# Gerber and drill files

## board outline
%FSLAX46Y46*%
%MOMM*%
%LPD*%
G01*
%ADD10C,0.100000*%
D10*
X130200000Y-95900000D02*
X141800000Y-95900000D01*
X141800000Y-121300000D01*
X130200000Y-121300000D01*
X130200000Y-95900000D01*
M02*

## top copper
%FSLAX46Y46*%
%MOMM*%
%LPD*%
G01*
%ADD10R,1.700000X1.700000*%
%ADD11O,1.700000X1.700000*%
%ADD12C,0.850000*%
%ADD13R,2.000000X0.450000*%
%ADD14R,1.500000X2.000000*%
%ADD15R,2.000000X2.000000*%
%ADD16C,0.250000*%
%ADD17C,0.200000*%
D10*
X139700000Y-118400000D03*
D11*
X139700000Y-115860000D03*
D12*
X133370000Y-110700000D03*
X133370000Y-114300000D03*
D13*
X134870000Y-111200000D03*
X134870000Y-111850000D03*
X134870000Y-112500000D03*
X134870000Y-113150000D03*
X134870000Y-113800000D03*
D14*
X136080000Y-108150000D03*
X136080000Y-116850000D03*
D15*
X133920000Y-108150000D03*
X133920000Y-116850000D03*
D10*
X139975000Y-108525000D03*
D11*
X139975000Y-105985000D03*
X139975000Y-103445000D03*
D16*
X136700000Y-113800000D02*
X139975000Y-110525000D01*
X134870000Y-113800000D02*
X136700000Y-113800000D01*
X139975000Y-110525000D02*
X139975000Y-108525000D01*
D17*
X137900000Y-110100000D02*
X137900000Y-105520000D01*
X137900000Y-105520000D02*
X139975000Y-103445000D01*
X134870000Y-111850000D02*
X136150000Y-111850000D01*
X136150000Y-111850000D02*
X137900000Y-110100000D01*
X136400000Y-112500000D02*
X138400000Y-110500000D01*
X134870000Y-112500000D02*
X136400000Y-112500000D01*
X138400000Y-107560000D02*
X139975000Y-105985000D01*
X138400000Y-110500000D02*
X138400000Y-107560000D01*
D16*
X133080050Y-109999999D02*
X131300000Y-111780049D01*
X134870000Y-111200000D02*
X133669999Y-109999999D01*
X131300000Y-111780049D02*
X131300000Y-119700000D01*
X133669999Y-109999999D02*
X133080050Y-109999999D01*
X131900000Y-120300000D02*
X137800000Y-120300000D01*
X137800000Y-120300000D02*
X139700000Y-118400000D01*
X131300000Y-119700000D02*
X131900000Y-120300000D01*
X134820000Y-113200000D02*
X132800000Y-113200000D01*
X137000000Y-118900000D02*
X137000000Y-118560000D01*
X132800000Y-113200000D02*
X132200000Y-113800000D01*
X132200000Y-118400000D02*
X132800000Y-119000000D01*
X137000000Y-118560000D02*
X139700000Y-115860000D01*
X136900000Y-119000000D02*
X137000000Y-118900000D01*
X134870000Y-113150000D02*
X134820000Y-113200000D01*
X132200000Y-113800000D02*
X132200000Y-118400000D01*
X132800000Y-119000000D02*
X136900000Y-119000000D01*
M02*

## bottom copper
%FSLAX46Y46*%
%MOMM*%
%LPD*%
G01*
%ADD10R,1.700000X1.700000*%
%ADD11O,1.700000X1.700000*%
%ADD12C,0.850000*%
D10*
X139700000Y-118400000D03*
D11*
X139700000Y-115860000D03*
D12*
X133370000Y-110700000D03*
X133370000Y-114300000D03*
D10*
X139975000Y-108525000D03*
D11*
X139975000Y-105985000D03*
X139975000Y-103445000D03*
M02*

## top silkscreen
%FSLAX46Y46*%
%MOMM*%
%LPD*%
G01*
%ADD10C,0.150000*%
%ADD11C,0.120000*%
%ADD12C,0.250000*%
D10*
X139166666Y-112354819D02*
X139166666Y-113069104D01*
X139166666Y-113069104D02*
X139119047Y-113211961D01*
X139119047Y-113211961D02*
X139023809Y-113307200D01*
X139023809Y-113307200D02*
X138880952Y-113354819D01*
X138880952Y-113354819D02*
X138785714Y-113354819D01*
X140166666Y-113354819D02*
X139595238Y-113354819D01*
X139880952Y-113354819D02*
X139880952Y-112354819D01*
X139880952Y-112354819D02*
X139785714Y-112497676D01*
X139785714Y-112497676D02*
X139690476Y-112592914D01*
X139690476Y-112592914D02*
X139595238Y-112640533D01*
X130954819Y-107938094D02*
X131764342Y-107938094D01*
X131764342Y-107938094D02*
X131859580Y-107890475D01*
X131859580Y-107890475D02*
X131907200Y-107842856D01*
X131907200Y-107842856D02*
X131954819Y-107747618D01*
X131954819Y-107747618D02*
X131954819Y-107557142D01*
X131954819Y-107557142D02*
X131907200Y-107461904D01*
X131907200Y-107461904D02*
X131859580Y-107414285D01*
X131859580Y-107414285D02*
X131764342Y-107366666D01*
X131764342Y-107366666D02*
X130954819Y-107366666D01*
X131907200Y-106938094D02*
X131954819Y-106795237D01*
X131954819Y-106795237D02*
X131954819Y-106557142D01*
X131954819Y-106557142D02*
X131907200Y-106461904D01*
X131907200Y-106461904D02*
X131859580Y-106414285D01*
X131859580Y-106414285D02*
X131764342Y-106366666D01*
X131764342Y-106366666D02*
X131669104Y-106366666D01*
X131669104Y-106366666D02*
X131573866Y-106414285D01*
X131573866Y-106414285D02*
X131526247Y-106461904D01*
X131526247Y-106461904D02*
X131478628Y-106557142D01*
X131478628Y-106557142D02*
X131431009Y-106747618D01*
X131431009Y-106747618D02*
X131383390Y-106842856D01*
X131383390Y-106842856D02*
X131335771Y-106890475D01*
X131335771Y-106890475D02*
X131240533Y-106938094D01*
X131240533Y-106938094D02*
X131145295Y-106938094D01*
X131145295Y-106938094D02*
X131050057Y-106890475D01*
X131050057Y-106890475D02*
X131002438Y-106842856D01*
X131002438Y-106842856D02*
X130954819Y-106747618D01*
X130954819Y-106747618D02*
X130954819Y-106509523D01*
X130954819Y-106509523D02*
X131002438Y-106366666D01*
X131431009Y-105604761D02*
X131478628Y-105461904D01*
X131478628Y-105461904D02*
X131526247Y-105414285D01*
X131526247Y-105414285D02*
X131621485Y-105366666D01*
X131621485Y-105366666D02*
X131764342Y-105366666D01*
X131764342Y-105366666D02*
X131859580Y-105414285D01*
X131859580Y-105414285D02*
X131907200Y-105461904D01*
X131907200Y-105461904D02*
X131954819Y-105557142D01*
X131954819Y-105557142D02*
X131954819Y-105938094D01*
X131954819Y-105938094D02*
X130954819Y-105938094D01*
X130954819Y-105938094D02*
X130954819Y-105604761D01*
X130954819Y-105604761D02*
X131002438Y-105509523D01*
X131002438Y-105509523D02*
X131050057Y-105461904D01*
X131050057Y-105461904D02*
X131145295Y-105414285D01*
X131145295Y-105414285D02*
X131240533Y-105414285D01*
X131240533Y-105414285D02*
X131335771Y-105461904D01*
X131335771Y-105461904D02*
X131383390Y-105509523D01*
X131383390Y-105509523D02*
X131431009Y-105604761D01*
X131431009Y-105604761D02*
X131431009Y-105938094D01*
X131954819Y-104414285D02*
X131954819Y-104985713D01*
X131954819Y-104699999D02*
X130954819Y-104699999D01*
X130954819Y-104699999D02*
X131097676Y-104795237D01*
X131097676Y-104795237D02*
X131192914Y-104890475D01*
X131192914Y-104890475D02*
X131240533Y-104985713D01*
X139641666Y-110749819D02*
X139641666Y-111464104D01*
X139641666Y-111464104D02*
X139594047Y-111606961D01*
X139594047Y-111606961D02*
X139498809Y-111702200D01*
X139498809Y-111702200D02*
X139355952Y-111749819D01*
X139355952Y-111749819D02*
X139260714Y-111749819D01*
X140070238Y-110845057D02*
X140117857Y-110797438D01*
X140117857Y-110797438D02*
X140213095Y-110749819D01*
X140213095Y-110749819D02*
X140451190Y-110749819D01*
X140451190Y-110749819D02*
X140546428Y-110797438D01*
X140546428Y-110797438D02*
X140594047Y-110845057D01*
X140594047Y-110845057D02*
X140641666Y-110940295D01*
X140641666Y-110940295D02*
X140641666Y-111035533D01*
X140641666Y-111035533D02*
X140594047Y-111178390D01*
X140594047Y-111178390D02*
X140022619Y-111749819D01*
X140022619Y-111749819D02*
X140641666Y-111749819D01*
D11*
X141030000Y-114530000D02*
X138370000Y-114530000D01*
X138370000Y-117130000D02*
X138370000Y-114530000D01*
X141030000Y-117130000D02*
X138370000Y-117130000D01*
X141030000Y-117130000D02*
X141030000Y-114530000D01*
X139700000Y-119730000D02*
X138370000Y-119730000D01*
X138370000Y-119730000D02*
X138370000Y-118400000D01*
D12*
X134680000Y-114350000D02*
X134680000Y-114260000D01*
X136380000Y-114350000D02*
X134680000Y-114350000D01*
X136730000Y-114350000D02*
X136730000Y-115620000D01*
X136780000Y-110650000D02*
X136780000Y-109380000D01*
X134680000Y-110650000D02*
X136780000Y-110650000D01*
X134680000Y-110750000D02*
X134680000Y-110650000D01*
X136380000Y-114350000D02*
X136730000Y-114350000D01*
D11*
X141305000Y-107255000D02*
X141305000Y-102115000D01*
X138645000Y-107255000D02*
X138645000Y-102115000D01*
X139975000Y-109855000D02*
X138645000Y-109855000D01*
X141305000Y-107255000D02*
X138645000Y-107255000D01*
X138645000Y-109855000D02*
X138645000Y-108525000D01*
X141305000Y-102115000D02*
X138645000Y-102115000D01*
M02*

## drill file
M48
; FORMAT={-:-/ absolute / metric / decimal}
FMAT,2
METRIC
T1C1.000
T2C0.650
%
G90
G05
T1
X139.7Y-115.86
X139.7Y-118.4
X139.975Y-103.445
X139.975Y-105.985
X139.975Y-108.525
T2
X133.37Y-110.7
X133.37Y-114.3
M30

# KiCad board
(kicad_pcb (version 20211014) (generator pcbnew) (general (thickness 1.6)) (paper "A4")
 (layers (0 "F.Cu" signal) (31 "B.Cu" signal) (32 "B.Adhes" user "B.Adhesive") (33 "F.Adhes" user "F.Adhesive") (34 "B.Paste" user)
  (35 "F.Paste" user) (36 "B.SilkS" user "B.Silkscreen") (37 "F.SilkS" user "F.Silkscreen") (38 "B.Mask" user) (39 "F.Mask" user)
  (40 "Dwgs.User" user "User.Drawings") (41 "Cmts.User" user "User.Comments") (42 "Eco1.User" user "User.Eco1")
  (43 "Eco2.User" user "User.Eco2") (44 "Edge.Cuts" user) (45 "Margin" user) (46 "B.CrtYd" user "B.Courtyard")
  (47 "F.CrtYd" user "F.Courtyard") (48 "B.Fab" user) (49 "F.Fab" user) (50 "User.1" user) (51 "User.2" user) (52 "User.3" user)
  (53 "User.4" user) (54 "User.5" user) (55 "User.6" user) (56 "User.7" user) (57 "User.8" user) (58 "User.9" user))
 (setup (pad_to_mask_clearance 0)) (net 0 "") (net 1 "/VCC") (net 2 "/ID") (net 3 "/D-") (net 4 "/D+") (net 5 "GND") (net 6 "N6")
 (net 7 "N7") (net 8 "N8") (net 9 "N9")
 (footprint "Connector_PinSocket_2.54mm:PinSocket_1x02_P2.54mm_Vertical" (layer "F.Cu") (at 139.7 118.4 180)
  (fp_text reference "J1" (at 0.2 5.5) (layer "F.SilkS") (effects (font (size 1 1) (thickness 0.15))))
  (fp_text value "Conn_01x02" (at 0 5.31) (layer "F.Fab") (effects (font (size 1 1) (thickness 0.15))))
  (fp_line (start -1.33 3.87) (end 1.33 3.87) (layer "F.SilkS") (width 0.12))
  (fp_line (start 1.33 1.27) (end 1.33 3.87) (layer "F.SilkS") (width 0.12))
  (fp_line (start -1.33 1.27) (end 1.33 1.27) (layer "F.SilkS") (width 0.12))
  (fp_line (start -1.33 1.27) (end -1.33 3.87) (layer "F.SilkS") (width 0.12))
  (fp_line (start 0 -1.33) (end 1.33 -1.33) (layer "F.SilkS") (width 0.12))
  (fp_line (start 1.33 -1.33) (end 1.33 0) (layer "F.SilkS") (width 0.12))
  (pad "1" thru_hole rect (at 0 0 180) (size 1.7 1.7) (drill 1) (layers *.Cu *.Mask) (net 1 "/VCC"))
  (pad "2" thru_hole oval (at 0 2.54 180) (size 1.7 1.7) (drill 1) (layers *.Cu *.Mask) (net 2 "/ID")))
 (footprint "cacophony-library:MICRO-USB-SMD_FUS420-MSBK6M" (layer "F.Cu") (at 135 112.5 -90)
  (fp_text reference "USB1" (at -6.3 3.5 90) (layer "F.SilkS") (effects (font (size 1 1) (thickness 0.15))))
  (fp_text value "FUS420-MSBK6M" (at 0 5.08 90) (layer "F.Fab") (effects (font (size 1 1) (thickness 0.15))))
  (fp_line (start 1.85 0.32) (end 1.76 0.32) (layer "F.SilkS") (width 0.25))
  (fp_line (start 1.85 -1.38) (end 1.85 0.32) (layer "F.SilkS") (width 0.25))
  (fp_line (start 1.85 -1.73) (end 3.12 -1.73) (layer "F.SilkS") (width 0.25))
  (fp_line (start -1.85 -1.78) (end -3.12 -1.78) (layer "F.SilkS") (width 0.25))
  (fp_line (start -1.85 0.32) (end -1.85 -1.78) (layer "F.SilkS") (width 0.25))
  (fp_line (start -1.75 0.32) (end -1.85 0.32) (layer "F.SilkS") (width 0.25))
  (fp_line (start 1.85 -1.38) (end 1.85 -1.73) (layer "F.SilkS") (width 0.25))
  (pad "" np_thru_hole circle (at -1.8 1.63 270) (size 0.85 0.85) (drill 0.65) (layers F&B.Cu *.Mask))
  (pad "" np_thru_hole circle (at 1.8 1.63 270) (size 0.85 0.85) (drill 0.65) (layers F&B.Cu *.Mask))
  (pad "1" smd rect (at -1.3 0.13 270) (size 0.45 2) (layers "F.Cu" "F.Paste" "F.Mask") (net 1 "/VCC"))
  (pad "2" smd rect (at -0.65 0.13 270) (size 0.45 2) (layers "F.Cu" "F.Paste" "F.Mask") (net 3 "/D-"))
  (pad "3" smd rect (at 0 0.13 270) (size 0.45 2) (layers "F.Cu" "F.Paste" "F.Mask") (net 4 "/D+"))
  (pad "4" smd rect (at 0.65 0.13 270) (size 0.45 2) (layers "F.Cu" "F.Paste" "F.Mask") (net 2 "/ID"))
  (pad "5" smd rect (at 1.3 0.13 270) (size 0.45 2) (layers "F.Cu" "F.Paste" "F.Mask") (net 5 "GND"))
  (pad "8" smd rect (at -4.35 -1.08 270) (size 2 1.5) (layers "F.Cu" "F.Paste" "F.Mask") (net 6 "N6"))
  (pad "9" smd rect (at 4.35 -1.08 270) (size 2 1.5) (layers "F.Cu" "F.Paste" "F.Mask") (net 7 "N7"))
  (pad "12" smd rect (at -4.35 1.08 270) (size 2 2) (layers "F.Cu" "F.Paste" "F.Mask") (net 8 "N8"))
  (pad "13" smd rect (at 4.35 1.08 270) (size 2 2) (layers "F.Cu" "F.Paste" "F.Mask") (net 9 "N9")))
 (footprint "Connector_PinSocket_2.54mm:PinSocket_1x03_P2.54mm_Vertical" (layer "F.Cu") (at 139.975 108.525 180)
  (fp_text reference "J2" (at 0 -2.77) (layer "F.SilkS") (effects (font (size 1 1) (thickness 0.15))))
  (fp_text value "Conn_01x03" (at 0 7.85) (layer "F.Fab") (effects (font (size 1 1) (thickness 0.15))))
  (fp_line (start -1.33 1.27) (end -1.33 6.41) (layer "F.SilkS") (width 0.12))
  (fp_line (start 1.33 1.27) (end 1.33 6.41) (layer "F.SilkS") (width 0.12))
  (fp_line (start 0 -1.33) (end 1.33 -1.33) (layer "F.SilkS") (width 0.12))
  (fp_line (start -1.33 1.27) (end 1.33 1.27) (layer "F.SilkS") (width 0.12))
  (fp_line (start 1.33 -1.33) (end 1.33 0) (layer "F.SilkS") (width 0.12))
  (fp_line (start -1.33 6.41) (end 1.33 6.41) (layer "F.SilkS") (width 0.12))
  (pad "1" thru_hole rect (at 0 0 180) (size 1.7 1.7) (drill 1) (layers *.Cu *.Mask) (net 5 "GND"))
  (pad "2" thru_hole oval (at 0 2.54 180) (size 1.7 1.7) (drill 1) (layers *.Cu *.Mask) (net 4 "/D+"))
  (pad "3" thru_hole oval (at 0 5.08 180) (size 1.7 1.7) (drill 1) (layers *.Cu *.Mask) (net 3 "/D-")))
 (gr_rect (start 130.2 121.3) (end 141.8 95.9) (layer "Edge.Cuts") (width 0.1) (fill none))
 (segment (start 136.7 113.8) (end 139.975 110.525) (width 0.25) (layer "F.Cu") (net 5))
 (segment (start 134.87 113.8) (end 136.7 113.8) (width 0.25) (layer "F.Cu") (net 5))
 (segment (start 139.975 110.525) (end 139.975 108.525) (width 0.25) (layer "F.Cu") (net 5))
 (segment (start 137.9 110.1) (end 137.9 105.52) (width 0.2) (layer "F.Cu") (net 3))
 (segment (start 137.9 105.52) (end 139.975 103.445) (width 0.2) (layer "F.Cu") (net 3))
 (segment (start 134.87 111.85) (end 136.15 111.85) (width 0.2) (layer "F.Cu") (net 3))
 (segment (start 136.15 111.85) (end 137.9 110.1) (width 0.2) (layer "F.Cu") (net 3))
 (segment (start 136.4 112.5) (end 138.4 110.5) (width 0.2) (layer "F.Cu") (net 4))
 (segment (start 134.87 112.5) (end 136.4 112.5) (width 0.2) (layer "F.Cu") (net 4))
 (segment (start 138.4 107.56) (end 139.975 105.985) (width 0.2) (layer "F.Cu") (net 4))
 (segment (start 138.4 110.5) (end 138.4 107.56) (width 0.2) (layer "F.Cu") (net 4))
 (segment (start 133.08005 109.999999) (end 131.3 111.780049) (width 0.25) (layer "F.Cu") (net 1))
 (segment (start 134.87 111.2) (end 133.669999 109.999999) (width 0.25) (layer "F.Cu") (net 1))
 (segment (start 131.3 111.780049) (end 131.3 119.7) (width 0.25) (layer "F.Cu") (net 1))
 (segment (start 133.669999 109.999999) (end 133.08005 109.999999) (width 0.25) (layer "F.Cu") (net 1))
 (segment (start 131.9 120.3) (end 137.8 120.3) (width 0.25) (layer "F.Cu") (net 1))
 (segment (start 137.8 120.3) (end 139.7 118.4) (width 0.25) (layer "F.Cu") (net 1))
 (segment (start 131.3 119.7) (end 131.9 120.3) (width 0.25) (layer "F.Cu") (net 1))
 (segment (start 134.82 113.2) (end 132.8 113.2) (width 0.25) (layer "F.Cu") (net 2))
 (segment (start 137 118.9) (end 137 118.56) (width 0.25) (layer "F.Cu") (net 2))
 (segment (start 132.8 113.2) (end 132.2 113.8) (width 0.25) (layer "F.Cu") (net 2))
 (segment (start 132.2 118.4) (end 132.8 119) (width 0.25) (layer "F.Cu") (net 2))
 (segment (start 137 118.56) (end 139.7 115.86) (width 0.25) (layer "F.Cu") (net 2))
 (segment (start 136.9 119) (end 137 118.9) (width 0.25) (layer "F.Cu") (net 2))
 (segment (start 134.87 113.15) (end 134.82 113.2) (width 0.25) (layer "F.Cu") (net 2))
 (segment (start 132.2 113.8) (end 132.2 118.4) (width 0.25) (layer "F.Cu") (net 2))
 (segment (start 132.8 119) (end 136.9 119) (width 0.25) (layer "F.Cu") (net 2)))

